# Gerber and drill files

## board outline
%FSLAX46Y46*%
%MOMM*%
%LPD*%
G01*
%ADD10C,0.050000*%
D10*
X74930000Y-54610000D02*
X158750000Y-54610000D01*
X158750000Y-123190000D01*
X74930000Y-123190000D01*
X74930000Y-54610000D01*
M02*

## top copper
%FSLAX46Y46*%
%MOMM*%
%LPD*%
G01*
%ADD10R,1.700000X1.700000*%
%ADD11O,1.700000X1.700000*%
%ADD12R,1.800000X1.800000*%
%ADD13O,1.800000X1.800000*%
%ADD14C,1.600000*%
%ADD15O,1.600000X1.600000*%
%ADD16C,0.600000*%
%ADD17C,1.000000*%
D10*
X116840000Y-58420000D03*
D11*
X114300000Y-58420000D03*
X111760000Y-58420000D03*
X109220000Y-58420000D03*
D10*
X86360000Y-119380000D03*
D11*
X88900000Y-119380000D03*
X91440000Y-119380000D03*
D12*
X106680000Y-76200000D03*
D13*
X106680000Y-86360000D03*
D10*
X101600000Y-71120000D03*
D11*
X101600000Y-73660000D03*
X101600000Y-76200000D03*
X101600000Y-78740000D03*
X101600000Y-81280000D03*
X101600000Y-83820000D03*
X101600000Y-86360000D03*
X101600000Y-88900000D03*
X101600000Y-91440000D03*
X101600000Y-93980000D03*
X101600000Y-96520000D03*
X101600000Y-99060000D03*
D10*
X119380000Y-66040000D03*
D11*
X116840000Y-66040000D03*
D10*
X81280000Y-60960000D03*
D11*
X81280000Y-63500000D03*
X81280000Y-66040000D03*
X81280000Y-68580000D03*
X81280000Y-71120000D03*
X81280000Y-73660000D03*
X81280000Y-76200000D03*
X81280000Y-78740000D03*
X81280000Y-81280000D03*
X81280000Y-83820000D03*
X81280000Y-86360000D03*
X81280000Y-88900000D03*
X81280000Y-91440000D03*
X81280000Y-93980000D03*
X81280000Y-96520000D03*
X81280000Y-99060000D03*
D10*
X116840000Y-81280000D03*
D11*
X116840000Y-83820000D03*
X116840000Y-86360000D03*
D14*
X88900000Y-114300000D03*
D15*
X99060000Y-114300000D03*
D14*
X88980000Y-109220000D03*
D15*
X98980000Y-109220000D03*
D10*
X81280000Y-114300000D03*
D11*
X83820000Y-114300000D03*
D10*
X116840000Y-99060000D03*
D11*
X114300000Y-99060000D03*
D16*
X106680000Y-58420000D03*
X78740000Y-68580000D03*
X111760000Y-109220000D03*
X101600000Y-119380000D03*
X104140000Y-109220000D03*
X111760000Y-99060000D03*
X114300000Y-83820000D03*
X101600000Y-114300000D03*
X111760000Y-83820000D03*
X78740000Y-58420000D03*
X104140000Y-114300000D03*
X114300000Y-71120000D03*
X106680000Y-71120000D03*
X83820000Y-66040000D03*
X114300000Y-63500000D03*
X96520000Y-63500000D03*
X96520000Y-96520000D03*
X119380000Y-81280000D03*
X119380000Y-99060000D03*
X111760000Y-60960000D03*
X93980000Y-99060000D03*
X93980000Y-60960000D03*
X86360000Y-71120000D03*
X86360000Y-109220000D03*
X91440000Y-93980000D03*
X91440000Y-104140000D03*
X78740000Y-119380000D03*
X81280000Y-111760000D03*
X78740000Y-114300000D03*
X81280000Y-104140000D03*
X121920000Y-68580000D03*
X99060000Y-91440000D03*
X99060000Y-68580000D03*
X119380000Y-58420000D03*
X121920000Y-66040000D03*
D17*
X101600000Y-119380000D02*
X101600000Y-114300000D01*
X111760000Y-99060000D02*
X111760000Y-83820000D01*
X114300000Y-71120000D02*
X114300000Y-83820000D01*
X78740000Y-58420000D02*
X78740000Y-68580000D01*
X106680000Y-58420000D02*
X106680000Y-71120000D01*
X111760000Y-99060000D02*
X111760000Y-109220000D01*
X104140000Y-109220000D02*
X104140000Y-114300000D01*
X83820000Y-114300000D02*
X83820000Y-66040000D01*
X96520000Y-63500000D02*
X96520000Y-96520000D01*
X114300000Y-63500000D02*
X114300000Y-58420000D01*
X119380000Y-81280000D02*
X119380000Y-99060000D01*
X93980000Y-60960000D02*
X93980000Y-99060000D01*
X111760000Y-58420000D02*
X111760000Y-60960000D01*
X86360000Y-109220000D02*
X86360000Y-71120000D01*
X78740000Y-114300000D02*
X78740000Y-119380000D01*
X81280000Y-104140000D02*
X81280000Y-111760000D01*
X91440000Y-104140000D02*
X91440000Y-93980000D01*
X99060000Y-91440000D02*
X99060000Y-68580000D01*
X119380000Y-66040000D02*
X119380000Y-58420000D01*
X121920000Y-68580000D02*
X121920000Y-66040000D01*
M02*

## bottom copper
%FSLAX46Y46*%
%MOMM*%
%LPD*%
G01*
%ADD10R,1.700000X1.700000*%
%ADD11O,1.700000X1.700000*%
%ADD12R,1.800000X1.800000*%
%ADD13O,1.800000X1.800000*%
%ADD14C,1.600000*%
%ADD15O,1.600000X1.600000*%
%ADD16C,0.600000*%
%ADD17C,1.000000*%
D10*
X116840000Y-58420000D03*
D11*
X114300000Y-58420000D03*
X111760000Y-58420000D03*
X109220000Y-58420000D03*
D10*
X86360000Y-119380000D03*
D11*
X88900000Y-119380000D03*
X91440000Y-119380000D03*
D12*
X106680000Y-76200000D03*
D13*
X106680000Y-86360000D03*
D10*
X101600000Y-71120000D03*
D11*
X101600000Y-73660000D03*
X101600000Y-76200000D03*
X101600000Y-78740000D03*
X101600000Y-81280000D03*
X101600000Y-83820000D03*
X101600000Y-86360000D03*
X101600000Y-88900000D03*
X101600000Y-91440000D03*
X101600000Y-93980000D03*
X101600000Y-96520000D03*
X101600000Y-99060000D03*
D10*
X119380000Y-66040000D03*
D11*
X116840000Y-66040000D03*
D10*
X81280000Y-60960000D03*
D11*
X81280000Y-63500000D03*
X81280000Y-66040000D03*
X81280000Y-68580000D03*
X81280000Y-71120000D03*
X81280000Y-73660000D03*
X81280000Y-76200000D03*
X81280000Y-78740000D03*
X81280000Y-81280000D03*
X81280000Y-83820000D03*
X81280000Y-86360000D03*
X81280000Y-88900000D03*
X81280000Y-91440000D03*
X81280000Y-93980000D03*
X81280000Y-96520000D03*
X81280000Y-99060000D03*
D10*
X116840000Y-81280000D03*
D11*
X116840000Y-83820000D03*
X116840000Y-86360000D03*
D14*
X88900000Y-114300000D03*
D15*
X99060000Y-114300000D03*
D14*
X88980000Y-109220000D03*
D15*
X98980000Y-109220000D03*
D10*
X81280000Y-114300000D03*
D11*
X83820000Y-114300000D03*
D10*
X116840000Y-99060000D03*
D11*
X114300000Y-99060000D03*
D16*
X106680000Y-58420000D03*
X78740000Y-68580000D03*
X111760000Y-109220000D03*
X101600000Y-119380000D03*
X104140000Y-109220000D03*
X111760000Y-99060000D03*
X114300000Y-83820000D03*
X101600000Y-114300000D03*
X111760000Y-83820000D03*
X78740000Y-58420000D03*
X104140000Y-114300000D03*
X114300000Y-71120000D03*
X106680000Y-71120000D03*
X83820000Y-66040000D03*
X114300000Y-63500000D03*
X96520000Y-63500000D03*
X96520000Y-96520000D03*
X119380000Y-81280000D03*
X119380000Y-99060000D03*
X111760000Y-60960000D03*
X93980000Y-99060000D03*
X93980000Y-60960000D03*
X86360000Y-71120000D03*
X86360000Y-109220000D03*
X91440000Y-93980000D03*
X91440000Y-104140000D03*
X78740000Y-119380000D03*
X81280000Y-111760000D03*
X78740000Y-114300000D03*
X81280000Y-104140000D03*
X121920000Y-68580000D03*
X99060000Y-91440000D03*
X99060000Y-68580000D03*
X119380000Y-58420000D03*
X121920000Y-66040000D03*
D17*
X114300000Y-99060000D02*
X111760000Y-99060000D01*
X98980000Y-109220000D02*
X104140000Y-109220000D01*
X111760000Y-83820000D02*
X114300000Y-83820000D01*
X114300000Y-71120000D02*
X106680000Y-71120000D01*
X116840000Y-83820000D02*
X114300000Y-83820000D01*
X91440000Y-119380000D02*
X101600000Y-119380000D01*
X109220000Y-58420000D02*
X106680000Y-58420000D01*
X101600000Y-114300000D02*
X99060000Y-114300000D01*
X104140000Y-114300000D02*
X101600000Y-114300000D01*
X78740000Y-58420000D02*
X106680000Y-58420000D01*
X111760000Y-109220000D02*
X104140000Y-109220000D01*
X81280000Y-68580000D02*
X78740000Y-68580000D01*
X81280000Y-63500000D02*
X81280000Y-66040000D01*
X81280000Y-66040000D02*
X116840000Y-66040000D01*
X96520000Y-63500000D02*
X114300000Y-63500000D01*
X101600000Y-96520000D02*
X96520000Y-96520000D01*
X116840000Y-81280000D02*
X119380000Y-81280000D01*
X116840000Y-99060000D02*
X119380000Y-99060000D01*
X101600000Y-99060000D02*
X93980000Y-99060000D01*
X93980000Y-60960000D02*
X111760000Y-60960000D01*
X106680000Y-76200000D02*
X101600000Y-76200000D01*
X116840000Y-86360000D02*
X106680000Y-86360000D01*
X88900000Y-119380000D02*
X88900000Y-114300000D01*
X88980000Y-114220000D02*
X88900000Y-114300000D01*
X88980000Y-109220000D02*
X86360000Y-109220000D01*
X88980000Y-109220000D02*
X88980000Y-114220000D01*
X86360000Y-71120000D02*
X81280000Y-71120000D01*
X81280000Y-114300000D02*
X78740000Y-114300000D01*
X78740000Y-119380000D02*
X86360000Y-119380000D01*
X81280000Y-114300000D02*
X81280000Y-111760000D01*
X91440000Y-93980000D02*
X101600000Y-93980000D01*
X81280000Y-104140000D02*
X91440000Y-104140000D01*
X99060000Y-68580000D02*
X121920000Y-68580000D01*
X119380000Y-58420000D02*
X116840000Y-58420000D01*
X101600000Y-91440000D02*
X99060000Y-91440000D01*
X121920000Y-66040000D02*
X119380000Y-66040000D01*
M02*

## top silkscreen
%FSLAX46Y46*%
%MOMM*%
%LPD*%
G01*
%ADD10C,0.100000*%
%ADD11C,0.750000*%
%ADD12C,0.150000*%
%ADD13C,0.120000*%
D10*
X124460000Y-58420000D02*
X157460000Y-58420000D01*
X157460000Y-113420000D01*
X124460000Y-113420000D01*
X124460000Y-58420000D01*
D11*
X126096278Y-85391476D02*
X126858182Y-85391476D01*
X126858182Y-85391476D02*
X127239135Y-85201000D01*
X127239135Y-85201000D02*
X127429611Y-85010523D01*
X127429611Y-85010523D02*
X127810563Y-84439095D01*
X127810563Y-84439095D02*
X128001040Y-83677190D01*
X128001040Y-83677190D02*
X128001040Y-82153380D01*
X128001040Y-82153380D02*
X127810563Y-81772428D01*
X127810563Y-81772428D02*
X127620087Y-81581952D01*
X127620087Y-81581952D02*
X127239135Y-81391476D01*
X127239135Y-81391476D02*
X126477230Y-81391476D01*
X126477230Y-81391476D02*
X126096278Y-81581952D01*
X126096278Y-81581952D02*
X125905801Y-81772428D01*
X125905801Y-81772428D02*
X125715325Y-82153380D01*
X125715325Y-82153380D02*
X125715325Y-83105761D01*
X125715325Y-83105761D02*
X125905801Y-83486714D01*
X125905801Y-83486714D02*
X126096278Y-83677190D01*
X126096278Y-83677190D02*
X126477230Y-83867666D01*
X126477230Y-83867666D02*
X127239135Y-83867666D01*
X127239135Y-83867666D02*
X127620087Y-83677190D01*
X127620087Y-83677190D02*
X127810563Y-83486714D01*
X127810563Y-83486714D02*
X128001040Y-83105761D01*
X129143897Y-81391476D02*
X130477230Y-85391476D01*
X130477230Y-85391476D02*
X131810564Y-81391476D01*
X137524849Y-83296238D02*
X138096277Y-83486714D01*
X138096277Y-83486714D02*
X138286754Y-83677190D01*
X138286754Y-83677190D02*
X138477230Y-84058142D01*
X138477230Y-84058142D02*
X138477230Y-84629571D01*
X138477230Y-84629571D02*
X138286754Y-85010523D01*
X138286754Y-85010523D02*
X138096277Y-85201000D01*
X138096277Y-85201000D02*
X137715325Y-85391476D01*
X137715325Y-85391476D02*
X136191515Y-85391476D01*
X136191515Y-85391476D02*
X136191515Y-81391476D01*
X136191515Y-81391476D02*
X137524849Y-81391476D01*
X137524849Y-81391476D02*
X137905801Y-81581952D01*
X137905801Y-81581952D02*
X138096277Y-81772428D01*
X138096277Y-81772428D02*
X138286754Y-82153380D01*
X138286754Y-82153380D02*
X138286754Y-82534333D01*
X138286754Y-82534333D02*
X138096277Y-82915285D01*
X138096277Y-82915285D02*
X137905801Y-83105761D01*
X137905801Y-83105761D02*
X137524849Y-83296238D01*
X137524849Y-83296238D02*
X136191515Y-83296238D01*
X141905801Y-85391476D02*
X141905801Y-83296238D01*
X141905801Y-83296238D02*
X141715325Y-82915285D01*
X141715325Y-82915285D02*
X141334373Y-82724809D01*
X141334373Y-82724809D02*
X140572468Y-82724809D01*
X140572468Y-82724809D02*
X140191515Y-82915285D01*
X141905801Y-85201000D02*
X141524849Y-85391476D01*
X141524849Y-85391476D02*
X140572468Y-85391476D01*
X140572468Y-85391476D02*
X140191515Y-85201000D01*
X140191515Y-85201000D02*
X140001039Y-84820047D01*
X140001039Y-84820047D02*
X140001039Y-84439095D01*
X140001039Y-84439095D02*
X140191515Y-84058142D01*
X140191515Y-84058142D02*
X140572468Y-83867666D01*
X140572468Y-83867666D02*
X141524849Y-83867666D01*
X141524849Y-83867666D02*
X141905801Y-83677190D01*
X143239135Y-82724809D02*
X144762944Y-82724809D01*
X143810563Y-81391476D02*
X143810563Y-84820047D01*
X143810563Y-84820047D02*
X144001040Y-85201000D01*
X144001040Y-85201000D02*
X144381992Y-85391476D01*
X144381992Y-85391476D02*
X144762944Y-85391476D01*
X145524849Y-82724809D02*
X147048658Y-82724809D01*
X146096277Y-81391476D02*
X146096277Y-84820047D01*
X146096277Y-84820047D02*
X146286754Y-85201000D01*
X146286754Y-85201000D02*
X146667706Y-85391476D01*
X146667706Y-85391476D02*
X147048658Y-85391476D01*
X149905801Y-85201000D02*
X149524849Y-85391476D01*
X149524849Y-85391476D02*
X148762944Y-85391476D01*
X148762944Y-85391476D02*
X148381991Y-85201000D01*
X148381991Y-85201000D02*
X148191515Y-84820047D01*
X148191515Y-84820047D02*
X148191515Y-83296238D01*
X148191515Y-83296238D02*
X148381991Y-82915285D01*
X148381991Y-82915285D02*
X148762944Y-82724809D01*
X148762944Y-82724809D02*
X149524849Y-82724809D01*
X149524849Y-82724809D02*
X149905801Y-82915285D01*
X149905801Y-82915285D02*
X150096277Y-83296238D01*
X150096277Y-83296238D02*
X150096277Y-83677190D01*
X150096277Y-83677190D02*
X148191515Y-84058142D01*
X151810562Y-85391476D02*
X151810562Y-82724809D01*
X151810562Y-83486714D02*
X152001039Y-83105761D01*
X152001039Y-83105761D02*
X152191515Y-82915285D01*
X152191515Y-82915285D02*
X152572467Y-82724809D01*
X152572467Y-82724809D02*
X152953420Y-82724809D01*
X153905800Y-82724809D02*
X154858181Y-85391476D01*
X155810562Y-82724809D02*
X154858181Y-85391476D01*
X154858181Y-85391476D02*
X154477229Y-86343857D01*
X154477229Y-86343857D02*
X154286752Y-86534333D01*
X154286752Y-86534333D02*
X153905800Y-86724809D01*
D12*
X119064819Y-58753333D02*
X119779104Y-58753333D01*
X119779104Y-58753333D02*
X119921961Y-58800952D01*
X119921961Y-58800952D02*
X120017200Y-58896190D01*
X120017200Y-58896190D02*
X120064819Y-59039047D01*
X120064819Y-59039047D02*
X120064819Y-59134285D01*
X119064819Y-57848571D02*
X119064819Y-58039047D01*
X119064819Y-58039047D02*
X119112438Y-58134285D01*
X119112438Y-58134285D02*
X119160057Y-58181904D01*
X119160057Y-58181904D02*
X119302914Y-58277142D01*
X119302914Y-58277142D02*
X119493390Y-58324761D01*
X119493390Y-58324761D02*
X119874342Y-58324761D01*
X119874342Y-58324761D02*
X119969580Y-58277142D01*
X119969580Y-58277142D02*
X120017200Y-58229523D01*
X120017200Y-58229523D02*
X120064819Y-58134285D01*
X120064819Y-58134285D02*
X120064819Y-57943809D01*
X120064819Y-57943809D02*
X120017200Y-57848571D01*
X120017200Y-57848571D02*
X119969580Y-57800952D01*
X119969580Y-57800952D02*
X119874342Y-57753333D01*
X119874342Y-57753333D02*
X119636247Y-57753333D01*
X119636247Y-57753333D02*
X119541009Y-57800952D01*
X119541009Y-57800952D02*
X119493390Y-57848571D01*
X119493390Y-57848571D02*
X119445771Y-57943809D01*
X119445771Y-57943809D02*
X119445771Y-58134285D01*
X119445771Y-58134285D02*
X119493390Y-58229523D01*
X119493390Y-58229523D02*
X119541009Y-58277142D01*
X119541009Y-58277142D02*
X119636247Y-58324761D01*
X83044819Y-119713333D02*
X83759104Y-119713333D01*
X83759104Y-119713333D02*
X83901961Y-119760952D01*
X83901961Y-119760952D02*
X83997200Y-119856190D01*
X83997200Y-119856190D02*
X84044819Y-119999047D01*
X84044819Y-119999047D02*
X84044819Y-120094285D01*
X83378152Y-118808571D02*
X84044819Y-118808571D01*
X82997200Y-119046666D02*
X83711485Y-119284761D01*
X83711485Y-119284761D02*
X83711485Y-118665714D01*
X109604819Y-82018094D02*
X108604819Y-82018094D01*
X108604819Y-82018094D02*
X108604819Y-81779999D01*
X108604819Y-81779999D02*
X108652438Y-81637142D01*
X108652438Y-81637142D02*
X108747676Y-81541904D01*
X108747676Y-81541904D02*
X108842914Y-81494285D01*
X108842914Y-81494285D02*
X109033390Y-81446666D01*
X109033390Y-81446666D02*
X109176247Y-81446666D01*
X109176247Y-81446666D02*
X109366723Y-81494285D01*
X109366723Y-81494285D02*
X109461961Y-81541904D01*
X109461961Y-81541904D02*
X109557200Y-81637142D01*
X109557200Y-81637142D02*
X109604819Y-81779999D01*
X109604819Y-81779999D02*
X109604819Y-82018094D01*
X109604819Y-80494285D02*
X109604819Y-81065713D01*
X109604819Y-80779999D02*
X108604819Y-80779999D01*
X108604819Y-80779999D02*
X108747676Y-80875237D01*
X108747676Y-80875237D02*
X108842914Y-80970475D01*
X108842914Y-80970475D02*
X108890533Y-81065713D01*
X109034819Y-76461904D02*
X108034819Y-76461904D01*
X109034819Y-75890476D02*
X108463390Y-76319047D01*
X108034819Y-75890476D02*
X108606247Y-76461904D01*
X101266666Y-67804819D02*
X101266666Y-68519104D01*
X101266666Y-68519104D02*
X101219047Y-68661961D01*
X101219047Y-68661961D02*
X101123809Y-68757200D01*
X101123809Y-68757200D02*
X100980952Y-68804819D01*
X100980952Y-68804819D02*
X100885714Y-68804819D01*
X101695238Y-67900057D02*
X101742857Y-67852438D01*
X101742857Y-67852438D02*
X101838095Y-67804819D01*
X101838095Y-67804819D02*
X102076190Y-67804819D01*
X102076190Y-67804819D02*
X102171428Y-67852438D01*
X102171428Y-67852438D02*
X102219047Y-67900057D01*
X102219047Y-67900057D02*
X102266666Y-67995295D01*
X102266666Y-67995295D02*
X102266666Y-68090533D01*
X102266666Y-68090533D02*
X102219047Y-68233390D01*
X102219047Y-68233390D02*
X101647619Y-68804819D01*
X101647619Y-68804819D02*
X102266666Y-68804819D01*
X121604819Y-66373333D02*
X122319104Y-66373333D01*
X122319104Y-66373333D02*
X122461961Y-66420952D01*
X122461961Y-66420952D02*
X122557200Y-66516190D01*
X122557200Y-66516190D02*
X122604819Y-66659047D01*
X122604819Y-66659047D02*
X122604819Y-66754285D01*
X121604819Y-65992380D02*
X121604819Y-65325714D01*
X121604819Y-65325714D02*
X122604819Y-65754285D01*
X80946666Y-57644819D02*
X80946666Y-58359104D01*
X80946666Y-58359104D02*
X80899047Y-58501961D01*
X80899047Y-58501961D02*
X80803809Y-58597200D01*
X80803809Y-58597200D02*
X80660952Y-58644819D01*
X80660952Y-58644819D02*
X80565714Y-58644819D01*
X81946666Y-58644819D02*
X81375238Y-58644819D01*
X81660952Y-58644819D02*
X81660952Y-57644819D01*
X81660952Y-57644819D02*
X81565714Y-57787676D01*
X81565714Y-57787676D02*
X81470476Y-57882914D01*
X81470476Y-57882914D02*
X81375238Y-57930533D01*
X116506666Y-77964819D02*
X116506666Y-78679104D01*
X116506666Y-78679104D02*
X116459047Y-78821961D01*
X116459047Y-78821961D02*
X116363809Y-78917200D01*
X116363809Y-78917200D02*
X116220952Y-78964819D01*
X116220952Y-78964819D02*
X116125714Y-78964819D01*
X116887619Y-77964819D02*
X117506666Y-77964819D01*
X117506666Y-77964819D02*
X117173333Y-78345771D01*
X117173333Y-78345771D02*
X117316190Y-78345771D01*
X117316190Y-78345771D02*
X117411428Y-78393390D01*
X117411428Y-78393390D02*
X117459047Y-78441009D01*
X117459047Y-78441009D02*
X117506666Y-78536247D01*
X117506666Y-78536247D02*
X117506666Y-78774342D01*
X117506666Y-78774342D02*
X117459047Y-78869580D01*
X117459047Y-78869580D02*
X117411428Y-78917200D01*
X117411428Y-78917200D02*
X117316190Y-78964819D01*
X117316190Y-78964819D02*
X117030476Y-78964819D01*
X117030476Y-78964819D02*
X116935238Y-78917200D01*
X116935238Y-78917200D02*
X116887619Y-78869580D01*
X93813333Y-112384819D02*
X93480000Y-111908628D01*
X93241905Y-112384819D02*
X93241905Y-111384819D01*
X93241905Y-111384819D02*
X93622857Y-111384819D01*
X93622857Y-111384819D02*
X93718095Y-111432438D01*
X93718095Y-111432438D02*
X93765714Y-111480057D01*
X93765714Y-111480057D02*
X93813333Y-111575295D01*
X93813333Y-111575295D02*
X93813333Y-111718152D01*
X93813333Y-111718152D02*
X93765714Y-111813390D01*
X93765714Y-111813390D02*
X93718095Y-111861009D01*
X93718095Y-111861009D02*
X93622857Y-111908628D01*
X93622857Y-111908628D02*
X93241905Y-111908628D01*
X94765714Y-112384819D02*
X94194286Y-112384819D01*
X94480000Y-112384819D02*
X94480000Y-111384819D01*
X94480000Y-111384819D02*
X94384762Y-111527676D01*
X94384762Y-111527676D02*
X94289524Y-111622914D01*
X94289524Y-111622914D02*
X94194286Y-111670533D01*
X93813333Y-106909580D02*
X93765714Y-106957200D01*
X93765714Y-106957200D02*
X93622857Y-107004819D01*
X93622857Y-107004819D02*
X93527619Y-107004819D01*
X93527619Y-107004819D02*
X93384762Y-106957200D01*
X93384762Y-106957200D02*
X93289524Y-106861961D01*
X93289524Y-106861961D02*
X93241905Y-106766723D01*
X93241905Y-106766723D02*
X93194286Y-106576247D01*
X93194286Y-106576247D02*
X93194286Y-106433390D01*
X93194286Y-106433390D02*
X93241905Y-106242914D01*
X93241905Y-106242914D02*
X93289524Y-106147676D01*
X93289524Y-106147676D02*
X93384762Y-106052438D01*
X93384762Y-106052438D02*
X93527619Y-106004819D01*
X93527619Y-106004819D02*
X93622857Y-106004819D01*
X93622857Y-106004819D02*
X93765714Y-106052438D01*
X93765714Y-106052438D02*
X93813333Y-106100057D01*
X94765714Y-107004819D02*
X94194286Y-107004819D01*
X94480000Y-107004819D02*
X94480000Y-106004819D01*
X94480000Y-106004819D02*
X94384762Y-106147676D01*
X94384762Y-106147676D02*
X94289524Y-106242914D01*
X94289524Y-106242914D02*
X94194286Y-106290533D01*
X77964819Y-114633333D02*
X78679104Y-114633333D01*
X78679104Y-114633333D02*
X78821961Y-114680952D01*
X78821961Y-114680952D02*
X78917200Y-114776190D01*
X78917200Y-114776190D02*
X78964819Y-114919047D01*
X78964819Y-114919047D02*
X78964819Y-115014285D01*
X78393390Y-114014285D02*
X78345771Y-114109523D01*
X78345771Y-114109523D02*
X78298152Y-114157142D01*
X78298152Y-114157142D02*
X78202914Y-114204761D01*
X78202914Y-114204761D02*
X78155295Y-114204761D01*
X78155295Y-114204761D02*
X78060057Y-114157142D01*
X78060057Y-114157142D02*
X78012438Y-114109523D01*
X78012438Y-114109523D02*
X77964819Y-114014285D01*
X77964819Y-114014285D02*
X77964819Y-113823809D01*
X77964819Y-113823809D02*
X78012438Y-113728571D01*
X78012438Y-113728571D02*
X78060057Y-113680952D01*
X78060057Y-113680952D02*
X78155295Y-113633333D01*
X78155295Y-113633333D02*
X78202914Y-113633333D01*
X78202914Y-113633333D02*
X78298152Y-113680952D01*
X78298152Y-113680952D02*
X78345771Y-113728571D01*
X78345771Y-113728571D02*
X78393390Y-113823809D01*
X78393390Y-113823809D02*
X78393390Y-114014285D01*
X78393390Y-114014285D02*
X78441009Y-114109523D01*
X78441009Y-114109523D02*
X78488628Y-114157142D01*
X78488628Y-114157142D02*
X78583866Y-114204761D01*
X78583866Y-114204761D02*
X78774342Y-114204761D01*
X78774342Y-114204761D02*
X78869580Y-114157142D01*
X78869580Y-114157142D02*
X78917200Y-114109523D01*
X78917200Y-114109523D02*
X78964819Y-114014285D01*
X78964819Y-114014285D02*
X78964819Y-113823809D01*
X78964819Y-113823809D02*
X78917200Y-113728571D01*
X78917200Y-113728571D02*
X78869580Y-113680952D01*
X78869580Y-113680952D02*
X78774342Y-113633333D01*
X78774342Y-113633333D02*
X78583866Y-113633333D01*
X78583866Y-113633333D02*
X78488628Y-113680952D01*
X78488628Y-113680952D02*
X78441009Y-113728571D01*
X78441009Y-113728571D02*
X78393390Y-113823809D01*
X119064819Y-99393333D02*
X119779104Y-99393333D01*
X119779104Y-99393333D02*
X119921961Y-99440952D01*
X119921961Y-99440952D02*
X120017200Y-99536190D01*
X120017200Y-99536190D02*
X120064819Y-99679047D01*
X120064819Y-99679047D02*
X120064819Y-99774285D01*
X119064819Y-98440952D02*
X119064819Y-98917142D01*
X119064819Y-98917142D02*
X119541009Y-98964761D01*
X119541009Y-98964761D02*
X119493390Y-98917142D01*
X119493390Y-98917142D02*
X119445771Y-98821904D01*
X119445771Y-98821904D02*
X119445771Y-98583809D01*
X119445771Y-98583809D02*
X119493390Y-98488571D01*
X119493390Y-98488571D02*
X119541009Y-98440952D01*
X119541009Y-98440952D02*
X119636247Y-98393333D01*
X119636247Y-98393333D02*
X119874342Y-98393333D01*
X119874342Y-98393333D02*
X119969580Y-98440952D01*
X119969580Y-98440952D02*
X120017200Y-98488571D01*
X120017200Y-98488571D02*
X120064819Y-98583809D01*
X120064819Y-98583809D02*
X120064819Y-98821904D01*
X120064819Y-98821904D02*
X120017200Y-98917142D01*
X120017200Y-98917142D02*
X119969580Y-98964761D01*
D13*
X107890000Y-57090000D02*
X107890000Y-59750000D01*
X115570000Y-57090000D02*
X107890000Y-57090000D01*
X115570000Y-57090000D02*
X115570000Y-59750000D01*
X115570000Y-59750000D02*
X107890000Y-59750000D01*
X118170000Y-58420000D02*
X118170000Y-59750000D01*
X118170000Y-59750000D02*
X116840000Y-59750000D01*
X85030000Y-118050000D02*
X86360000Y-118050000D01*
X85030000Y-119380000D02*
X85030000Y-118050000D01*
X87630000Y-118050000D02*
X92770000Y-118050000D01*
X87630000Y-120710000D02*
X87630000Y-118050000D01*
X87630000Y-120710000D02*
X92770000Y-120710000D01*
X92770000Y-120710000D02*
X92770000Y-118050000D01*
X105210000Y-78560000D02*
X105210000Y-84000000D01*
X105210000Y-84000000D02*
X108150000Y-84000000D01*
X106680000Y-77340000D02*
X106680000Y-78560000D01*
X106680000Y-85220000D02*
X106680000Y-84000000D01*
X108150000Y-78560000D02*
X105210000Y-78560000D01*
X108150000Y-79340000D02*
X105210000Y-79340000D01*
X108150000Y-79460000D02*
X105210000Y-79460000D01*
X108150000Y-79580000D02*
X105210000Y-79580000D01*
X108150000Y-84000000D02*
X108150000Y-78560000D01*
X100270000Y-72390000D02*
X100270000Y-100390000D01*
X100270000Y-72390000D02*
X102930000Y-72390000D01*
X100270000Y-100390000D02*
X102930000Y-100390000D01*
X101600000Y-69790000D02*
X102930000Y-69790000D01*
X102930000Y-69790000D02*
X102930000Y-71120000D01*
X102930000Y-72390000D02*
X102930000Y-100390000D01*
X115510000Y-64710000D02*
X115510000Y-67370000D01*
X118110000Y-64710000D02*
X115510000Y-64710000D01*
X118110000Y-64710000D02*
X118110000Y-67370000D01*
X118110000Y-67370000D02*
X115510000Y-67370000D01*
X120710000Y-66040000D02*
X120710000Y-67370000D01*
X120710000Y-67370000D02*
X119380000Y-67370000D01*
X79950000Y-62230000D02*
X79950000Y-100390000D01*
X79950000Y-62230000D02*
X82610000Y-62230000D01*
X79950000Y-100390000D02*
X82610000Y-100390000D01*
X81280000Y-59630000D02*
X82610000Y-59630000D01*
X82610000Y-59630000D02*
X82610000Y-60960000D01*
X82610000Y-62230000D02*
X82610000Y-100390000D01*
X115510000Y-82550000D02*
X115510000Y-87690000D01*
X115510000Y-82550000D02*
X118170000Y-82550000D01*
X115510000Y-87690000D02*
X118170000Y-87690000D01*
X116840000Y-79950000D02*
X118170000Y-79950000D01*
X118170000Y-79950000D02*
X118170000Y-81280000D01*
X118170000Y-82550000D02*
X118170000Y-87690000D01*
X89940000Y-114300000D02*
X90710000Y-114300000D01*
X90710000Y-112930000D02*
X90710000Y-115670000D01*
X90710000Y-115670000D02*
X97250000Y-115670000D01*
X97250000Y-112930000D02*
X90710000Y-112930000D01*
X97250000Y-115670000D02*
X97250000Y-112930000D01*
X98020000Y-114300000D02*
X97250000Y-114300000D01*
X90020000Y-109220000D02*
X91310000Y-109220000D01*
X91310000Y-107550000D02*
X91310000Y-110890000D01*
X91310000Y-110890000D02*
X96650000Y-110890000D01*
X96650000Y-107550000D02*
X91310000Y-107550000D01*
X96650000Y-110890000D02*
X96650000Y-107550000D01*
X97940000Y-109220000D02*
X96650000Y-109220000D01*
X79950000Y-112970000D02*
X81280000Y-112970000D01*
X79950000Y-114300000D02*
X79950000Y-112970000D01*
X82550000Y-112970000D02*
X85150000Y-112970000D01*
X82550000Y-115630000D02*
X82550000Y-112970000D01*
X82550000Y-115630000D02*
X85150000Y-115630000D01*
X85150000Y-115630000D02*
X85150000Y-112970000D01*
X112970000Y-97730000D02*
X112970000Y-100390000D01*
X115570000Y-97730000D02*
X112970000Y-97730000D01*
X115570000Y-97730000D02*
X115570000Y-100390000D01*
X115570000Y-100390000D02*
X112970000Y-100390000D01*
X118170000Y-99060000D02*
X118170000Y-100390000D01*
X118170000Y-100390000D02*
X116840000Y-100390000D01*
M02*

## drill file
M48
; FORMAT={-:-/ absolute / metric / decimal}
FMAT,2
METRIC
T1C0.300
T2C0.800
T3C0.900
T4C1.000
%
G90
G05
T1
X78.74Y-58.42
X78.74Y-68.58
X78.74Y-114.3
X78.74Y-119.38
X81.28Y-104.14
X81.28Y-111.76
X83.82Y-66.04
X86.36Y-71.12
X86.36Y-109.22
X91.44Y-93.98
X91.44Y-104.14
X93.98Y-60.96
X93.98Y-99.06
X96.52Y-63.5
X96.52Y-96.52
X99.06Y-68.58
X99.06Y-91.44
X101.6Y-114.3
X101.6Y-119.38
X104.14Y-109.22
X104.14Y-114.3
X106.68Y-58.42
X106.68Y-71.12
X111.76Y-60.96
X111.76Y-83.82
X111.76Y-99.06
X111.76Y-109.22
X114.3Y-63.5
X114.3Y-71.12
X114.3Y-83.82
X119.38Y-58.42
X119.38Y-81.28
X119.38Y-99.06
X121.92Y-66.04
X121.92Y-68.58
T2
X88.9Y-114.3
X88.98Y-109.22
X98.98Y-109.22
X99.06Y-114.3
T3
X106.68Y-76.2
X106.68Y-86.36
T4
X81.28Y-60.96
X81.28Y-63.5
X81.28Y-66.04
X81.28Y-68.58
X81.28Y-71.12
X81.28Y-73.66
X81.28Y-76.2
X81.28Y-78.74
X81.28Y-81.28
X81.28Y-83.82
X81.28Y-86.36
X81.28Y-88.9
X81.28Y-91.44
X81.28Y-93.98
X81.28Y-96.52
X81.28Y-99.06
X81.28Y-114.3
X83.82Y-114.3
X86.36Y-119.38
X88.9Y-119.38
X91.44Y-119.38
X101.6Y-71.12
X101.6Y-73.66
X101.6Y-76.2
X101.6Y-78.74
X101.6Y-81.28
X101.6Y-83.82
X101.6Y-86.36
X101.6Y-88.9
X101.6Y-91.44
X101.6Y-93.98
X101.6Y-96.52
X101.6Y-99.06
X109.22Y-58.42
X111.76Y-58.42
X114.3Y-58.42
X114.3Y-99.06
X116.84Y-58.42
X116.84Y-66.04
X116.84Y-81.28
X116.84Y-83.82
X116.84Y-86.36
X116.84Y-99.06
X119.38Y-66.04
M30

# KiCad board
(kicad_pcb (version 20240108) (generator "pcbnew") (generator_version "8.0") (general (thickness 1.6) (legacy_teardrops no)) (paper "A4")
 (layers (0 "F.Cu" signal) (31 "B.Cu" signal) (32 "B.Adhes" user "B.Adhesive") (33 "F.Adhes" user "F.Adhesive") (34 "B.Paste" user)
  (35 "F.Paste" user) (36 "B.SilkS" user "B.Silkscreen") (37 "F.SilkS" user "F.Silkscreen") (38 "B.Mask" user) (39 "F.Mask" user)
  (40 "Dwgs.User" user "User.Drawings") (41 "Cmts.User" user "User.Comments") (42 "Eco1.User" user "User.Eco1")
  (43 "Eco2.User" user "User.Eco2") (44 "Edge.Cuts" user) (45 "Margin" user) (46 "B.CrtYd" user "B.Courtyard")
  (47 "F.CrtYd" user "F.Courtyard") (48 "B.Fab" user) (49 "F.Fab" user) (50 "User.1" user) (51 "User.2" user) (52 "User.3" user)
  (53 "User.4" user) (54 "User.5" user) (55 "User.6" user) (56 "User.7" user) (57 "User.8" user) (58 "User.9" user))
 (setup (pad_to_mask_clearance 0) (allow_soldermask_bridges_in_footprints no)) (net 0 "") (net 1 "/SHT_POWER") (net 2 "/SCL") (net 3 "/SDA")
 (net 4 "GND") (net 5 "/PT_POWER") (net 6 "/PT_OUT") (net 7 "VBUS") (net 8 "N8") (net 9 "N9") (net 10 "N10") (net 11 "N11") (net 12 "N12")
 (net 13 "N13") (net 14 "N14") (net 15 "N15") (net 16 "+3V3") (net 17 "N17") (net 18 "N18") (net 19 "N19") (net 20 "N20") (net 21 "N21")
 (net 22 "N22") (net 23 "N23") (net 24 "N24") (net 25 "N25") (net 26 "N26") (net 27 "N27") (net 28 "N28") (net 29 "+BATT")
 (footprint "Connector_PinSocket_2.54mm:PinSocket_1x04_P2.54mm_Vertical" (layer "F.Cu") (at 116.84 58.42 -90)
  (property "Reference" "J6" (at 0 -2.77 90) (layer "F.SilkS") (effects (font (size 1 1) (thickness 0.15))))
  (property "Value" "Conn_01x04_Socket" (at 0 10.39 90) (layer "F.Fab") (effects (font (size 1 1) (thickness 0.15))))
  (fp_line (start -1.33 8.95) (end 1.33 8.95) (stroke (width 0.12) (type solid)) (layer "F.SilkS"))
  (fp_line (start -1.33 1.27) (end -1.33 8.95) (stroke (width 0.12) (type solid)) (layer "F.SilkS"))
  (fp_line (start -1.33 1.27) (end 1.33 1.27) (stroke (width 0.12) (type solid)) (layer "F.SilkS"))
  (fp_line (start 1.33 1.27) (end 1.33 8.95) (stroke (width 0.12) (type solid)) (layer "F.SilkS"))
  (fp_line (start 0 -1.33) (end 1.33 -1.33) (stroke (width 0.12) (type solid)) (layer "F.SilkS"))
  (fp_line (start 1.33 -1.33) (end 1.33 0) (stroke (width 0.12) (type solid)) (layer "F.SilkS"))
  (pad "1" thru_hole rect (at 0 0 270) (size 1.7 1.7) (drill 1) (layers "*.Cu" "*.Mask") (remove_unused_layers no) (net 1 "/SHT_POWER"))
  (pad "2" thru_hole oval (at 0 2.54 270) (size 1.7 1.7) (drill 1) (layers "*.Cu" "*.Mask") (remove_unused_layers no) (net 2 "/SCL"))
  (pad "3" thru_hole oval (at 0 5.08 270) (size 1.7 1.7) (drill 1) (layers "*.Cu" "*.Mask") (remove_unused_layers no) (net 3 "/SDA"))
  (pad "4" thru_hole oval (at 0 7.62 270) (size 1.7 1.7) (drill 1) (layers "*.Cu" "*.Mask") (remove_unused_layers no) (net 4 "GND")))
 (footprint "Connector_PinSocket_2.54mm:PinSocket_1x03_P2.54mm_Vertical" (layer "F.Cu") (at 86.36 119.38 90)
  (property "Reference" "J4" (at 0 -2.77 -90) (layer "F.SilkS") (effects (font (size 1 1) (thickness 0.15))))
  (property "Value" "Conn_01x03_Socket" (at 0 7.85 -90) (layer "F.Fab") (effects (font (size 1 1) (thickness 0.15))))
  (fp_line (start 1.33 -1.33) (end 1.33 0) (stroke (width 0.12) (type solid)) (layer "F.SilkS"))
  (fp_line (start 0 -1.33) (end 1.33 -1.33) (stroke (width 0.12) (type solid)) (layer "F.SilkS"))
  (fp_line (start 1.33 1.27) (end 1.33 6.41) (stroke (width 0.12) (type solid)) (layer "F.SilkS"))
  (fp_line (start -1.33 1.27) (end 1.33 1.27) (stroke (width 0.12) (type solid)) (layer "F.SilkS"))
  (fp_line (start -1.33 1.27) (end -1.33 6.41) (stroke (width 0.12) (type solid)) (layer "F.SilkS"))
  (fp_line (start -1.33 6.41) (end 1.33 6.41) (stroke (width 0.12) (type solid)) (layer "F.SilkS"))
  (pad "1" thru_hole rect (at 0 0 90) (size 1.7 1.7) (drill 1) (layers "*.Cu" "*.Mask") (remove_unused_layers no) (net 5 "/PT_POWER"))
  (pad "2" thru_hole oval (at 0 2.54 90) (size 1.7 1.7) (drill 1) (layers "*.Cu" "*.Mask") (remove_unused_layers no) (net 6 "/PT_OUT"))
  (pad "3" thru_hole oval (at 0 5.08 90) (size 1.7 1.7) (drill 1) (layers "*.Cu" "*.Mask") (remove_unused_layers no) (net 4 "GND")))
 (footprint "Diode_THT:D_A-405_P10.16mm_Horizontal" (layer "F.Cu") (at 106.68 76.2 -90)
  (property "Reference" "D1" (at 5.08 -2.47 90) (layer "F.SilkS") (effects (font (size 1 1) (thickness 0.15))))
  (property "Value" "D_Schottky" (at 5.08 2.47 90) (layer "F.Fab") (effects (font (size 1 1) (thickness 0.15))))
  (fp_line (start 2.36 1.47) (end 7.8 1.47) (stroke (width 0.12) (type solid)) (layer "F.SilkS"))
  (fp_line (start 7.8 1.47) (end 7.8 -1.47) (stroke (width 0.12) (type solid)) (layer "F.SilkS"))
  (fp_line (start 1.14 0) (end 2.36 0) (stroke (width 0.12) (type solid)) (layer "F.SilkS"))
  (fp_line (start 9.02 0) (end 7.8 0) (stroke (width 0.12) (type solid)) (layer "F.SilkS"))
  (fp_line (start 2.36 -1.47) (end 2.36 1.47) (stroke (width 0.12) (type solid)) (layer "F.SilkS"))
  (fp_line (start 3.14 -1.47) (end 3.14 1.47) (stroke (width 0.12) (type solid)) (layer "F.SilkS"))
  (fp_line (start 3.26 -1.47) (end 3.26 1.47) (stroke (width 0.12) (type solid)) (layer "F.SilkS"))
  (fp_line (start 3.38 -1.47) (end 3.38 1.47) (stroke (width 0.12) (type solid)) (layer "F.SilkS"))
  (fp_line (start 7.8 -1.47) (end 2.36 -1.47) (stroke (width 0.12) (type solid)) (layer "F.SilkS"))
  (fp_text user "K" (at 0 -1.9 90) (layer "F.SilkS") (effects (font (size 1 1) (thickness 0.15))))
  (pad "1" thru_hole rect (at 0 0 270) (size 1.8 1.8) (drill 0.9) (layers "*.Cu" "*.Mask") (remove_unused_layers no) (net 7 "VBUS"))
  (pad "2" thru_hole oval (at 10.16 0 270) (size 1.8 1.8) (drill 0.9) (layers "*.Cu" "*.Mask") (remove_unused_layers no) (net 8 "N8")))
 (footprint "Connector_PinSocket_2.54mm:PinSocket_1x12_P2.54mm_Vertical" (layer "F.Cu") (at 101.6 71.12)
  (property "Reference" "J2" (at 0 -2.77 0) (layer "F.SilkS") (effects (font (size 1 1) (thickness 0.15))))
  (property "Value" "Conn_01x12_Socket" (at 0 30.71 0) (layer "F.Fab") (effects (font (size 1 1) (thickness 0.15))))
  (fp_line (start -1.33 1.27) (end -1.33 29.27) (stroke (width 0.12) (type solid)) (layer "F.SilkS"))
  (fp_line (start -1.33 1.27) (end 1.33 1.27) (stroke (width 0.12) (type solid)) (layer "F.SilkS"))
  (fp_line (start -1.33 29.27) (end 1.33 29.27) (stroke (width 0.12) (type solid)) (layer "F.SilkS"))
  (fp_line (start 0 -1.33) (end 1.33 -1.33) (stroke (width 0.12) (type solid)) (layer "F.SilkS"))
  (fp_line (start 1.33 -1.33) (end 1.33 0) (stroke (width 0.12) (type solid)) (layer "F.SilkS"))
  (fp_line (start 1.33 1.27) (end 1.33 29.27) (stroke (width 0.12) (type solid)) (layer "F.SilkS"))
  (pad "1" thru_hole rect (at 0 0) (size 1.7 1.7) (drill 1) (layers "*.Cu" "*.Mask") (remove_unused_layers no) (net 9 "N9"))
  (pad "2" thru_hole oval (at 0 2.54) (size 1.7 1.7) (drill 1) (layers "*.Cu" "*.Mask") (remove_unused_layers no) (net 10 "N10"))
  (pad "3" thru_hole oval (at 0 5.08) (size 1.7 1.7) (drill 1) (layers "*.Cu" "*.Mask") (remove_unused_layers no) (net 7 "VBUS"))
  (pad "4" thru_hole oval (at 0 7.62) (size 1.7 1.7) (drill 1) (layers "*.Cu" "*.Mask") (remove_unused_layers no) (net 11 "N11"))
  (pad "5" thru_hole oval (at 0 10.16) (size 1.7 1.7) (drill 1) (layers "*.Cu" "*.Mask") (remove_unused_layers no) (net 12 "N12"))
  (pad "6" thru_hole oval (at 0 12.7) (size 1.7 1.7) (drill 1) (layers "*.Cu" "*.Mask") (remove_unused_layers no) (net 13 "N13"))
  (pad "7" thru_hole oval (at 0 15.24) (size 1.7 1.7) (drill 1) (layers "*.Cu" "*.Mask") (remove_unused_layers no) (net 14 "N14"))
  (pad "8" thru_hole oval (at 0 17.78) (size 1.7 1.7) (drill 1) (layers "*.Cu" "*.Mask") (remove_unused_layers no) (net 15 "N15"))
  (pad "9" thru_hole oval (at 0 20.32) (size 1.7 1.7) (drill 1) (layers "*.Cu" "*.Mask") (remove_unused_layers no) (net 1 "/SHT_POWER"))
  (pad "10" thru_hole oval (at 0 22.86) (size 1.7 1.7) (drill 1) (layers "*.Cu" "*.Mask") (remove_unused_layers no) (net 5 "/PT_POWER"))
  (pad "11" thru_hole oval (at 0 25.4) (size 1.7 1.7) (drill 1) (layers "*.Cu" "*.Mask") (remove_unused_layers no) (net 2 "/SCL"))
  (pad "12" thru_hole oval (at 0 27.94) (size 1.7 1.7) (drill 1) (layers "*.Cu" "*.Mask") (remove_unused_layers no) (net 3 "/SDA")))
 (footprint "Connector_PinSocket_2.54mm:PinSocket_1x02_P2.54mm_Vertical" (layer "F.Cu") (at 119.38 66.04 -90)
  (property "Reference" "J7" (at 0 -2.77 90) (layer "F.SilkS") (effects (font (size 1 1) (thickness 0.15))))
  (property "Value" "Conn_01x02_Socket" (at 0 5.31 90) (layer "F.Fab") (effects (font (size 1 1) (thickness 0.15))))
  (fp_line (start -1.33 3.87) (end 1.33 3.87) (stroke (width 0.12) (type solid)) (layer "F.SilkS"))
  (fp_line (start -1.33 1.27) (end -1.33 3.87) (stroke (width 0.12) (type solid)) (layer "F.SilkS"))
  (fp_line (start -1.33 1.27) (end 1.33 1.27) (stroke (width 0.12) (type solid)) (layer "F.SilkS"))
  (fp_line (start 1.33 1.27) (end 1.33 3.87) (stroke (width 0.12) (type solid)) (layer "F.SilkS"))
  (fp_line (start 0 -1.33) (end 1.33 -1.33) (stroke (width 0.12) (type solid)) (layer "F.SilkS"))
  (fp_line (start 1.33 -1.33) (end 1.33 0) (stroke (width 0.12) (type solid)) (layer "F.SilkS"))
  (pad "1" thru_hole rect (at 0 0 270) (size 1.7 1.7) (drill 1) (layers "*.Cu" "*.Mask") (remove_unused_layers no) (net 1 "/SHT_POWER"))
  (pad "2" thru_hole oval (at 0 2.54 270) (size 1.7 1.7) (drill 1) (layers "*.Cu" "*.Mask") (remove_unused_layers no) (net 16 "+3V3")))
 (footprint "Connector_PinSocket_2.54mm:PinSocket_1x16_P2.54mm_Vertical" (layer "F.Cu") (at 81.28 60.96)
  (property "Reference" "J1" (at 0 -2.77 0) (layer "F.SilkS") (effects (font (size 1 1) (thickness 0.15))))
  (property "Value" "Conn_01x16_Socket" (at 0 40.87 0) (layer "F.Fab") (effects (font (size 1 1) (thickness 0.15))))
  (fp_line (start -1.33 1.27) (end -1.33 39.43) (stroke (width 0.12) (type solid)) (layer "F.SilkS"))
  (fp_line (start -1.33 1.27) (end 1.33 1.27) (stroke (width 0.12) (type solid)) (layer "F.SilkS"))
  (fp_line (start -1.33 39.43) (end 1.33 39.43) (stroke (width 0.12) (type solid)) (layer "F.SilkS"))
  (fp_line (start 0 -1.33) (end 1.33 -1.33) (stroke (width 0.12) (type solid)) (layer "F.SilkS"))
  (fp_line (start 1.33 -1.33) (end 1.33 0) (stroke (width 0.12) (type solid)) (layer "F.SilkS"))
  (fp_line (start 1.33 1.27) (end 1.33 39.43) (stroke (width 0.12) (type solid)) (layer "F.SilkS"))
  (pad "1" thru_hole rect (at 0 0) (size 1.7 1.7) (drill 1) (layers "*.Cu" "*.Mask") (remove_unused_layers no) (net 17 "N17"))
  (pad "2" thru_hole oval (at 0 2.54) (size 1.7 1.7) (drill 1) (layers "*.Cu" "*.Mask") (remove_unused_layers no) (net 16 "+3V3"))
  (pad "3" thru_hole oval (at 0 5.08) (size 1.7 1.7) (drill 1) (layers "*.Cu" "*.Mask") (remove_unused_layers no) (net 16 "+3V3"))
  (pad "4" thru_hole oval (at 0 7.62) (size 1.7 1.7) (drill 1) (layers "*.Cu" "*.Mask") (remove_unused_layers no) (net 4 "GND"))
  (pad "5" thru_hole oval (at 0 10.16) (size 1.7 1.7) (drill 1) (layers "*.Cu" "*.Mask") (remove_unused_layers no) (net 6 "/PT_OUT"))
  (pad "6" thru_hole oval (at 0 12.7) (size 1.7 1.7) (drill 1) (layers "*.Cu" "*.Mask") (remove_unused_layers no) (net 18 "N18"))
  (pad "7" thru_hole oval (at 0 15.24) (size 1.7 1.7) (drill 1) (layers "*.Cu" "*.Mask") (remove_unused_layers no) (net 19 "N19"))
  (pad "8" thru_hole oval (at 0 17.78) (size 1.7 1.7) (drill 1) (layers "*.Cu" "*.Mask") (remove_unused_layers no) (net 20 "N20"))
  (pad "9" thru_hole oval (at 0 20.32) (size 1.7 1.7) (drill 1) (layers "*.Cu" "*.Mask") (remove_unused_layers no) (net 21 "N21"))
  (pad "10" thru_hole oval (at 0 22.86) (size 1.7 1.7) (drill 1) (layers "*.Cu" "*.Mask") (remove_unused_layers no) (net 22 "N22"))
  (pad "11" thru_hole oval (at 0 25.4) (size 1.7 1.7) (drill 1) (layers "*.Cu" "*.Mask") (remove_unused_layers no) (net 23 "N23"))
  (pad "12" thru_hole oval (at 0 27.94) (size 1.7 1.7) (drill 1) (layers "*.Cu" "*.Mask") (remove_unused_layers no) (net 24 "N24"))
  (pad "13" thru_hole oval (at 0 30.48) (size 1.7 1.7) (drill 1) (layers "*.Cu" "*.Mask") (remove_unused_layers no) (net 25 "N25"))
  (pad "14" thru_hole oval (at 0 33.02) (size 1.7 1.7) (drill 1) (layers "*.Cu" "*.Mask") (remove_unused_layers no) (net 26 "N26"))
  (pad "15" thru_hole oval (at 0 35.56) (size 1.7 1.7) (drill 1) (layers "*.Cu" "*.Mask") (remove_unused_layers no) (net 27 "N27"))
  (pad "16" thru_hole oval (at 0 38.1) (size 1.7 1.7) (drill 1) (layers "*.Cu" "*.Mask") (remove_unused_layers no) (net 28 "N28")))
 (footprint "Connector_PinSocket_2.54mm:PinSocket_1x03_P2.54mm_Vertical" (layer "F.Cu") (at 116.84 81.28)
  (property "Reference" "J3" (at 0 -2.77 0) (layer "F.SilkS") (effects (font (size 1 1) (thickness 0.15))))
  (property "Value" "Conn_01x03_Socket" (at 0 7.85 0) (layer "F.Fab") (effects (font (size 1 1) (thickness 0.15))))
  (fp_line (start -1.33 1.27) (end -1.33 6.41) (stroke (width 0.12) (type solid)) (layer "F.SilkS"))
  (fp_line (start -1.33 1.27) (end 1.33 1.27) (stroke (width 0.12) (type solid)) (layer "F.SilkS"))
  (fp_line (start -1.33 6.41) (end 1.33 6.41) (stroke (width 0.12) (type solid)) (layer "F.SilkS"))
  (fp_line (start 0 -1.33) (end 1.33 -1.33) (stroke (width 0.12) (type solid)) (layer "F.SilkS"))
  (fp_line (start 1.33 -1.33) (end 1.33 0) (stroke (width 0.12) (type solid)) (layer "F.SilkS"))
  (fp_line (start 1.33 1.27) (end 1.33 6.41) (stroke (width 0.12) (type solid)) (layer "F.SilkS"))
  (pad "1" thru_hole rect (at 0 0) (size 1.7 1.7) (drill 1) (layers "*.Cu" "*.Mask") (remove_unused_layers no) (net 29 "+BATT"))
  (pad "2" thru_hole oval (at 0 2.54) (size 1.7 1.7) (drill 1) (layers "*.Cu" "*.Mask") (remove_unused_layers no) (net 4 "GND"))
  (pad "3" thru_hole oval (at 0 5.08) (size 1.7 1.7) (drill 1) (layers "*.Cu" "*.Mask") (remove_unused_layers no) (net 8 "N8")))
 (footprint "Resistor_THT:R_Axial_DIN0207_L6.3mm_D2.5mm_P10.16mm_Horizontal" (layer "F.Cu") (at 88.9 114.3)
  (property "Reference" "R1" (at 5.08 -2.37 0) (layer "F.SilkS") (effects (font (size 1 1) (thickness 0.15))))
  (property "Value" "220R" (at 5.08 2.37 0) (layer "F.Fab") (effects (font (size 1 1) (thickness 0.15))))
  (fp_line (start 1.04 0) (end 1.81 0) (stroke (width 0.12) (type solid)) (layer "F.SilkS"))
  (fp_line (start 1.81 -1.37) (end 1.81 1.37) (stroke (width 0.12) (type solid)) (layer "F.SilkS"))
  (fp_line (start 1.81 1.37) (end 8.35 1.37) (stroke (width 0.12) (type solid)) (layer "F.SilkS"))
  (fp_line (start 8.35 -1.37) (end 1.81 -1.37) (stroke (width 0.12) (type solid)) (layer "F.SilkS"))
  (fp_line (start 8.35 1.37) (end 8.35 -1.37) (stroke (width 0.12) (type solid)) (layer "F.SilkS"))
  (fp_line (start 9.12 0) (end 8.35 0) (stroke (width 0.12) (type solid)) (layer "F.SilkS"))
  (pad "1" thru_hole circle (at 0 0) (size 1.6 1.6) (drill 0.8) (layers "*.Cu" "*.Mask") (remove_unused_layers no) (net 6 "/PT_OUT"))
  (pad "2" thru_hole oval (at 10.16 0) (size 1.6 1.6) (drill 0.8) (layers "*.Cu" "*.Mask") (remove_unused_layers no) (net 4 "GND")))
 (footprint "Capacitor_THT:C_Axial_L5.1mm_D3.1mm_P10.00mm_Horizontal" (layer "F.Cu") (at 88.98 109.22)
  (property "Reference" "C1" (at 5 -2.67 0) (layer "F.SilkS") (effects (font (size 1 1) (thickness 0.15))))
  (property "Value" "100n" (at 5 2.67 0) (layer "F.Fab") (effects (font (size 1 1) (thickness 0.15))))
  (fp_line (start 1.04 0) (end 2.33 0) (stroke (width 0.12) (type solid)) (layer "F.SilkS"))
  (fp_line (start 2.33 -1.67) (end 2.33 1.67) (stroke (width 0.12) (type solid)) (layer "F.SilkS"))
  (fp_line (start 2.33 1.67) (end 7.67 1.67) (stroke (width 0.12) (type solid)) (layer "F.SilkS"))
  (fp_line (start 7.67 -1.67) (end 2.33 -1.67) (stroke (width 0.12) (type solid)) (layer "F.SilkS"))
  (fp_line (start 7.67 1.67) (end 7.67 -1.67) (stroke (width 0.12) (type solid)) (layer "F.SilkS"))
  (fp_line (start 8.96 0) (end 7.67 0) (stroke (width 0.12) (type solid)) (layer "F.SilkS"))
  (pad "1" thru_hole circle (at 0 0) (size 1.6 1.6) (drill 0.8) (layers "*.Cu" "*.Mask") (remove_unused_layers no) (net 6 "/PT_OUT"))
  (pad "2" thru_hole oval (at 10 0) (size 1.6 1.6) (drill 0.8) (layers "*.Cu" "*.Mask") (remove_unused_layers no) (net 4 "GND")))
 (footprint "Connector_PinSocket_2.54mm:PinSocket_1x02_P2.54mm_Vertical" (layer "F.Cu") (at 81.28 114.3 90)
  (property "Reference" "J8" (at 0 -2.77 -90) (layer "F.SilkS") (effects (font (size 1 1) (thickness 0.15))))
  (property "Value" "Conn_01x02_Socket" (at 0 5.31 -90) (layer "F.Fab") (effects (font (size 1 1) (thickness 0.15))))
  (fp_line (start 1.33 -1.33) (end 1.33 0) (stroke (width 0.12) (type solid)) (layer "F.SilkS"))
  (fp_line (start 0 -1.33) (end 1.33 -1.33) (stroke (width 0.12) (type solid)) (layer "F.SilkS"))
  (fp_line (start 1.33 1.27) (end 1.33 3.87) (stroke (width 0.12) (type solid)) (layer "F.SilkS"))
  (fp_line (start -1.33 1.27) (end 1.33 1.27) (stroke (width 0.12) (type solid)) (layer "F.SilkS"))
  (fp_line (start -1.33 1.27) (end -1.33 3.87) (stroke (width 0.12) (type solid)) (layer "F.SilkS"))
  (fp_line (start -1.33 3.87) (end 1.33 3.87) (stroke (width 0.12) (type solid)) (layer "F.SilkS"))
  (pad "1" thru_hole rect (at 0 0 90) (size 1.7 1.7) (drill 1) (layers "*.Cu" "*.Mask") (remove_unused_layers no) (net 5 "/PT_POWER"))
  (pad "2" thru_hole oval (at 0 2.54 90) (size 1.7 1.7) (drill 1) (layers "*.Cu" "*.Mask") (remove_unused_layers no) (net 16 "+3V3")))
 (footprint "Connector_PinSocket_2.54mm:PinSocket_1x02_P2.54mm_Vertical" (layer "F.Cu") (at 116.84 99.06 -90)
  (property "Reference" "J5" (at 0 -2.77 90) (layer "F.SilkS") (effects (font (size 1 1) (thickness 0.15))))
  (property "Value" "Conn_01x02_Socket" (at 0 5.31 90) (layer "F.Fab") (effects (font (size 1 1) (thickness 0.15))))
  (fp_line (start -1.33 3.87) (end 1.33 3.87) (stroke (width 0.12) (type solid)) (layer "F.SilkS"))
  (fp_line (start -1.33 1.27) (end -1.33 3.87) (stroke (width 0.12) (type solid)) (layer "F.SilkS"))
  (fp_line (start -1.33 1.27) (end 1.33 1.27) (stroke (width 0.12) (type solid)) (layer "F.SilkS"))
  (fp_line (start 1.33 1.27) (end 1.33 3.87) (stroke (width 0.12) (type solid)) (layer "F.SilkS"))
  (fp_line (start 0 -1.33) (end 1.33 -1.33) (stroke (width 0.12) (type solid)) (layer "F.SilkS"))
  (fp_line (start 1.33 -1.33) (end 1.33 0) (stroke (width 0.12) (type solid)) (layer "F.SilkS"))
  (pad "1" thru_hole rect (at 0 0 270) (size 1.7 1.7) (drill 1) (layers "*.Cu" "*.Mask") (remove_unused_layers no) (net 29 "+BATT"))
  (pad "2" thru_hole oval (at 0 2.54 270) (size 1.7 1.7) (drill 1) (layers "*.Cu" "*.Mask") (remove_unused_layers no) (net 4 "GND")))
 (gr_rect (start 124.46 58.42) (end 157.46 113.42) (stroke (width 0.1) (type default)) (fill none) (layer "F.SilkS"))
 (gr_rect (start 74.93 54.61) (end 158.75 123.19) (stroke (width 0.05) (type default)) (fill none) (layer "Edge.Cuts"))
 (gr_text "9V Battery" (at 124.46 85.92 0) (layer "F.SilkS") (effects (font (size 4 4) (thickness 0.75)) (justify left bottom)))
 (segment (start 101.6 119.38) (end 101.6 114.3) (width 1) (layer "F.Cu") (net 4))
 (segment (start 111.76 99.06) (end 111.76 83.82) (width 1) (layer "F.Cu") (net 4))
 (segment (start 114.3 71.12) (end 114.3 83.82) (width 1) (layer "F.Cu") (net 4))
 (segment (start 78.74 58.42) (end 78.74 68.58) (width 1) (layer "F.Cu") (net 4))
 (segment (start 106.68 58.42) (end 106.68 71.12) (width 1) (layer "F.Cu") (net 4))
 (segment (start 111.76 99.06) (end 111.76 109.22) (width 1) (layer "F.Cu") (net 4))
 (segment (start 104.14 109.22) (end 104.14 114.3) (width 1) (layer "F.Cu") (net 4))
 (via (at 106.68 58.42) (size 0.6) (drill 0.3) (layers "F.Cu" "B.Cu") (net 4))
 (via (at 78.74 68.58) (size 0.6) (drill 0.3) (layers "F.Cu" "B.Cu") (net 4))
 (via (at 111.76 109.22) (size 0.6) (drill 0.3) (layers "F.Cu" "B.Cu") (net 4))
 (via (at 101.6 119.38) (size 0.6) (drill 0.3) (layers "F.Cu" "B.Cu") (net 4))
 (via (at 104.14 109.22) (size 0.6) (drill 0.3) (layers "F.Cu" "B.Cu") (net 4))
 (via (at 111.76 99.06) (size 0.6) (drill 0.3) (layers "F.Cu" "B.Cu") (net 4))
 (via (at 114.3 83.82) (size 0.6) (drill 0.3) (layers "F.Cu" "B.Cu") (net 4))
 (via (at 101.6 114.3) (size 0.6) (drill 0.3) (layers "F.Cu" "B.Cu") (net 4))
 (via (at 111.76 83.82) (size 0.6) (drill 0.3) (layers "F.Cu" "B.Cu") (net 4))
 (via (at 78.74 58.42) (size 0.6) (drill 0.3) (layers "F.Cu" "B.Cu") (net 4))
 (via (at 104.14 114.3) (size 0.6) (drill 0.3) (layers "F.Cu" "B.Cu") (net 4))
 (via (at 114.3 71.12) (size 0.6) (drill 0.3) (layers "F.Cu" "B.Cu") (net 4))
 (via (at 106.68 71.12) (size 0.6) (drill 0.3) (layers "F.Cu" "B.Cu") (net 4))
 (segment (start 114.3 99.06) (end 111.76 99.06) (width 1) (layer "B.Cu") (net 4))
 (segment (start 98.98 109.22) (end 104.14 109.22) (width 1) (layer "B.Cu") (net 4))
 (segment (start 111.76 83.82) (end 114.3 83.82) (width 1) (layer "B.Cu") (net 4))
 (segment (start 114.3 71.12) (end 106.68 71.12) (width 1) (layer "B.Cu") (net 4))
 (segment (start 116.84 83.82) (end 114.3 83.82) (width 1) (layer "B.Cu") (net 4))
 (segment (start 91.44 119.38) (end 101.6 119.38) (width 1) (layer "B.Cu") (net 4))
 (segment (start 109.22 58.42) (end 106.68 58.42) (width 1) (layer "B.Cu") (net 4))
 (segment (start 101.6 114.3) (end 99.06 114.3) (width 1) (layer "B.Cu") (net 4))
 (segment (start 104.14 114.3) (end 101.6 114.3) (width 1) (layer "B.Cu") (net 4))
 (segment (start 78.74 58.42) (end 106.68 58.42) (width 1) (layer "B.Cu") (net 4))
 (segment (start 111.76 109.22) (end 104.14 109.22) (width 1) (layer "B.Cu") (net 4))
 (segment (start 81.28 68.58) (end 78.74 68.58) (width 1) (layer "B.Cu") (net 4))
 (segment (start 83.82 114.3) (end 83.82 66.04) (width 1) (layer "F.Cu") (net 16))
 (via (at 83.82 66.04) (size 0.6) (drill 0.3) (layers "F.Cu" "B.Cu") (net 16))
 (segment (start 81.28 63.5) (end 81.28 66.04) (width 1) (layer "B.Cu") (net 16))
 (segment (start 81.28 66.04) (end 116.84 66.04) (width 1) (layer "B.Cu") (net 16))
 (segment (start 96.52 63.5) (end 96.52 96.52) (width 1) (layer "F.Cu") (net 2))
 (segment (start 114.3 63.5) (end 114.3 58.42) (width 1) (layer "F.Cu") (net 2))
 (via (at 114.3 63.5) (size 0.6) (drill 0.3) (layers "F.Cu" "B.Cu") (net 2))
 (via (at 96.52 63.5) (size 0.6) (drill 0.3) (layers "F.Cu" "B.Cu") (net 2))
 (via (at 96.52 96.52) (size 0.6) (drill 0.3) (layers "F.Cu" "B.Cu") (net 2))
 (segment (start 96.52 63.5) (end 114.3 63.5) (width 1) (layer "B.Cu") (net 2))
 (segment (start 101.6 96.52) (end 96.52 96.52) (width 1) (layer "B.Cu") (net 2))
 (segment (start 119.38 81.28) (end 119.38 99.06) (width 1) (layer "F.Cu") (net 29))
 (via (at 119.38 81.28) (size 0.6) (drill 0.3) (layers "F.Cu" "B.Cu") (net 29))
 (via (at 119.38 99.06) (size 0.6) (drill 0.3) (layers "F.Cu" "B.Cu") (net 29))
 (segment (start 116.84 81.28) (end 119.38 81.28) (width 1) (layer "B.Cu") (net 29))
 (segment (start 116.84 99.06) (end 119.38 99.06) (width 1) (layer "B.Cu") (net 29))
 (segment (start 93.98 60.96) (end 93.98 99.06) (width 1) (layer "F.Cu") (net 3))
 (segment (start 111.76 58.42) (end 111.76 60.96) (width 1) (layer "F.Cu") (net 3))
 (via (at 111.76 60.96) (size 0.6) (drill 0.3) (layers "F.Cu" "B.Cu") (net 3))
 (via (at 93.98 99.06) (size 0.6) (drill 0.3) (layers "F.Cu" "B.Cu") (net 3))
 (via (at 93.98 60.96) (size 0.6) (drill 0.3) (layers "F.Cu" "B.Cu") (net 3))
 (segment (start 101.6 99.06) (end 93.98 99.06) (width 1) (layer "B.Cu") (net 3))
 (segment (start 93.98 60.96) (end 111.76 60.96) (width 1) (layer "B.Cu") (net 3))
 (segment (start 106.68 76.2) (end 101.6 76.2) (width 1) (layer "B.Cu") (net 7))
 (segment (start 116.84 86.36) (end 106.68 86.36) (width 1) (layer "B.Cu") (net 8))
 (segment (start 86.36 109.22) (end 86.36 71.12) (width 1) (layer "F.Cu") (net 6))
 (via (at 86.36 71.12) (size 0.6) (drill 0.3) (layers "F.Cu" "B.Cu") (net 6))
 (via (at 86.36 109.22) (size 0.6) (drill 0.3) (layers "F.Cu" "B.Cu") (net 6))
 (segment (start 88.9 119.38) (end 88.9 114.3) (width 1) (layer "B.Cu") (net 6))
 (segment (start 88.98 114.22) (end 88.9 114.3) (width 1) (layer "B.Cu") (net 6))
 (segment (start 88.98 109.22) (end 86.36 109.22) (width 1) (layer "B.Cu") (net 6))
 (segment (start 88.98 109.22) (end 88.98 114.22) (width 1) (layer "B.Cu") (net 6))
 (segment (start 86.36 71.12) (end 81.28 71.12) (width 1) (layer "B.Cu") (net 6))
 (segment (start 78.74 114.3) (end 78.74 119.38) (width 1) (layer "F.Cu") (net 5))
 (segment (start 81.28 104.14) (end 81.28 111.76) (width 1) (layer "F.Cu") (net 5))
 (segment (start 91.44 104.14) (end 91.44 93.98) (width 1) (layer "F.Cu") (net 5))
 (via (at 91.44 93.98) (size 0.6) (drill 0.3) (layers "F.Cu" "B.Cu") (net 5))
 (via (at 91.44 104.14) (size 0.6) (drill 0.3) (layers "F.Cu" "B.Cu") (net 5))
 (via (at 78.74 119.38) (size 0.6) (drill 0.3) (layers "F.Cu" "B.Cu") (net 5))
 (via (at 81.28 111.76) (size 0.6) (drill 0.3) (layers "F.Cu" "B.Cu") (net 5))
 (via (at 78.74 114.3) (size 0.6) (drill 0.3) (layers "F.Cu" "B.Cu") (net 5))
 (via (at 81.28 104.14) (size 0.6) (drill 0.3) (layers "F.Cu" "B.Cu") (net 5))
 (segment (start 81.28 114.3) (end 78.74 114.3) (width 1) (layer "B.Cu") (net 5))
 (segment (start 78.74 119.38) (end 86.36 119.38) (width 1) (layer "B.Cu") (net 5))
 (segment (start 81.28 114.3) (end 81.28 111.76) (width 1) (layer "B.Cu") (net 5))
 (segment (start 91.44 93.98) (end 101.6 93.98) (width 1) (layer "B.Cu") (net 5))
 (segment (start 81.28 104.14) (end 91.44 104.14) (width 1) (layer "B.Cu") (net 5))
 (segment (start 99.06 91.44) (end 99.06 68.58) (width 1) (layer "F.Cu") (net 1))
 (segment (start 119.38 66.04) (end 119.38 58.42) (width 1) (layer "F.Cu") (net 1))
 (segment (start 121.92 68.58) (end 121.92 66.04) (width 1) (layer "F.Cu") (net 1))
 (via (at 121.92 68.58) (size 0.6) (drill 0.3) (layers "F.Cu" "B.Cu") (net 1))
 (via (at 99.06 91.44) (size 0.6) (drill 0.3) (layers "F.Cu" "B.Cu") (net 1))
 (via (at 99.06 68.58) (size 0.6) (drill 0.3) (layers "F.Cu" "B.Cu") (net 1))
 (via (at 119.38 58.42) (size 0.6) (drill 0.3) (layers "F.Cu" "B.Cu") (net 1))
 (via (at 121.92 66.04) (size 0.6) (drill 0.3) (layers "F.Cu" "B.Cu") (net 1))
 (segment (start 99.06 68.58) (end 121.92 68.58) (width 1) (layer "B.Cu") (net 1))
 (segment (start 119.38 58.42) (end 116.84 58.42) (width 1) (layer "B.Cu") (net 1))
 (segment (start 101.6 91.44) (end 99.06 91.44) (width 1) (layer "B.Cu") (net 1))
 (segment (start 121.92 66.04) (end 119.38 66.04) (width 1) (layer "B.Cu") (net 1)))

